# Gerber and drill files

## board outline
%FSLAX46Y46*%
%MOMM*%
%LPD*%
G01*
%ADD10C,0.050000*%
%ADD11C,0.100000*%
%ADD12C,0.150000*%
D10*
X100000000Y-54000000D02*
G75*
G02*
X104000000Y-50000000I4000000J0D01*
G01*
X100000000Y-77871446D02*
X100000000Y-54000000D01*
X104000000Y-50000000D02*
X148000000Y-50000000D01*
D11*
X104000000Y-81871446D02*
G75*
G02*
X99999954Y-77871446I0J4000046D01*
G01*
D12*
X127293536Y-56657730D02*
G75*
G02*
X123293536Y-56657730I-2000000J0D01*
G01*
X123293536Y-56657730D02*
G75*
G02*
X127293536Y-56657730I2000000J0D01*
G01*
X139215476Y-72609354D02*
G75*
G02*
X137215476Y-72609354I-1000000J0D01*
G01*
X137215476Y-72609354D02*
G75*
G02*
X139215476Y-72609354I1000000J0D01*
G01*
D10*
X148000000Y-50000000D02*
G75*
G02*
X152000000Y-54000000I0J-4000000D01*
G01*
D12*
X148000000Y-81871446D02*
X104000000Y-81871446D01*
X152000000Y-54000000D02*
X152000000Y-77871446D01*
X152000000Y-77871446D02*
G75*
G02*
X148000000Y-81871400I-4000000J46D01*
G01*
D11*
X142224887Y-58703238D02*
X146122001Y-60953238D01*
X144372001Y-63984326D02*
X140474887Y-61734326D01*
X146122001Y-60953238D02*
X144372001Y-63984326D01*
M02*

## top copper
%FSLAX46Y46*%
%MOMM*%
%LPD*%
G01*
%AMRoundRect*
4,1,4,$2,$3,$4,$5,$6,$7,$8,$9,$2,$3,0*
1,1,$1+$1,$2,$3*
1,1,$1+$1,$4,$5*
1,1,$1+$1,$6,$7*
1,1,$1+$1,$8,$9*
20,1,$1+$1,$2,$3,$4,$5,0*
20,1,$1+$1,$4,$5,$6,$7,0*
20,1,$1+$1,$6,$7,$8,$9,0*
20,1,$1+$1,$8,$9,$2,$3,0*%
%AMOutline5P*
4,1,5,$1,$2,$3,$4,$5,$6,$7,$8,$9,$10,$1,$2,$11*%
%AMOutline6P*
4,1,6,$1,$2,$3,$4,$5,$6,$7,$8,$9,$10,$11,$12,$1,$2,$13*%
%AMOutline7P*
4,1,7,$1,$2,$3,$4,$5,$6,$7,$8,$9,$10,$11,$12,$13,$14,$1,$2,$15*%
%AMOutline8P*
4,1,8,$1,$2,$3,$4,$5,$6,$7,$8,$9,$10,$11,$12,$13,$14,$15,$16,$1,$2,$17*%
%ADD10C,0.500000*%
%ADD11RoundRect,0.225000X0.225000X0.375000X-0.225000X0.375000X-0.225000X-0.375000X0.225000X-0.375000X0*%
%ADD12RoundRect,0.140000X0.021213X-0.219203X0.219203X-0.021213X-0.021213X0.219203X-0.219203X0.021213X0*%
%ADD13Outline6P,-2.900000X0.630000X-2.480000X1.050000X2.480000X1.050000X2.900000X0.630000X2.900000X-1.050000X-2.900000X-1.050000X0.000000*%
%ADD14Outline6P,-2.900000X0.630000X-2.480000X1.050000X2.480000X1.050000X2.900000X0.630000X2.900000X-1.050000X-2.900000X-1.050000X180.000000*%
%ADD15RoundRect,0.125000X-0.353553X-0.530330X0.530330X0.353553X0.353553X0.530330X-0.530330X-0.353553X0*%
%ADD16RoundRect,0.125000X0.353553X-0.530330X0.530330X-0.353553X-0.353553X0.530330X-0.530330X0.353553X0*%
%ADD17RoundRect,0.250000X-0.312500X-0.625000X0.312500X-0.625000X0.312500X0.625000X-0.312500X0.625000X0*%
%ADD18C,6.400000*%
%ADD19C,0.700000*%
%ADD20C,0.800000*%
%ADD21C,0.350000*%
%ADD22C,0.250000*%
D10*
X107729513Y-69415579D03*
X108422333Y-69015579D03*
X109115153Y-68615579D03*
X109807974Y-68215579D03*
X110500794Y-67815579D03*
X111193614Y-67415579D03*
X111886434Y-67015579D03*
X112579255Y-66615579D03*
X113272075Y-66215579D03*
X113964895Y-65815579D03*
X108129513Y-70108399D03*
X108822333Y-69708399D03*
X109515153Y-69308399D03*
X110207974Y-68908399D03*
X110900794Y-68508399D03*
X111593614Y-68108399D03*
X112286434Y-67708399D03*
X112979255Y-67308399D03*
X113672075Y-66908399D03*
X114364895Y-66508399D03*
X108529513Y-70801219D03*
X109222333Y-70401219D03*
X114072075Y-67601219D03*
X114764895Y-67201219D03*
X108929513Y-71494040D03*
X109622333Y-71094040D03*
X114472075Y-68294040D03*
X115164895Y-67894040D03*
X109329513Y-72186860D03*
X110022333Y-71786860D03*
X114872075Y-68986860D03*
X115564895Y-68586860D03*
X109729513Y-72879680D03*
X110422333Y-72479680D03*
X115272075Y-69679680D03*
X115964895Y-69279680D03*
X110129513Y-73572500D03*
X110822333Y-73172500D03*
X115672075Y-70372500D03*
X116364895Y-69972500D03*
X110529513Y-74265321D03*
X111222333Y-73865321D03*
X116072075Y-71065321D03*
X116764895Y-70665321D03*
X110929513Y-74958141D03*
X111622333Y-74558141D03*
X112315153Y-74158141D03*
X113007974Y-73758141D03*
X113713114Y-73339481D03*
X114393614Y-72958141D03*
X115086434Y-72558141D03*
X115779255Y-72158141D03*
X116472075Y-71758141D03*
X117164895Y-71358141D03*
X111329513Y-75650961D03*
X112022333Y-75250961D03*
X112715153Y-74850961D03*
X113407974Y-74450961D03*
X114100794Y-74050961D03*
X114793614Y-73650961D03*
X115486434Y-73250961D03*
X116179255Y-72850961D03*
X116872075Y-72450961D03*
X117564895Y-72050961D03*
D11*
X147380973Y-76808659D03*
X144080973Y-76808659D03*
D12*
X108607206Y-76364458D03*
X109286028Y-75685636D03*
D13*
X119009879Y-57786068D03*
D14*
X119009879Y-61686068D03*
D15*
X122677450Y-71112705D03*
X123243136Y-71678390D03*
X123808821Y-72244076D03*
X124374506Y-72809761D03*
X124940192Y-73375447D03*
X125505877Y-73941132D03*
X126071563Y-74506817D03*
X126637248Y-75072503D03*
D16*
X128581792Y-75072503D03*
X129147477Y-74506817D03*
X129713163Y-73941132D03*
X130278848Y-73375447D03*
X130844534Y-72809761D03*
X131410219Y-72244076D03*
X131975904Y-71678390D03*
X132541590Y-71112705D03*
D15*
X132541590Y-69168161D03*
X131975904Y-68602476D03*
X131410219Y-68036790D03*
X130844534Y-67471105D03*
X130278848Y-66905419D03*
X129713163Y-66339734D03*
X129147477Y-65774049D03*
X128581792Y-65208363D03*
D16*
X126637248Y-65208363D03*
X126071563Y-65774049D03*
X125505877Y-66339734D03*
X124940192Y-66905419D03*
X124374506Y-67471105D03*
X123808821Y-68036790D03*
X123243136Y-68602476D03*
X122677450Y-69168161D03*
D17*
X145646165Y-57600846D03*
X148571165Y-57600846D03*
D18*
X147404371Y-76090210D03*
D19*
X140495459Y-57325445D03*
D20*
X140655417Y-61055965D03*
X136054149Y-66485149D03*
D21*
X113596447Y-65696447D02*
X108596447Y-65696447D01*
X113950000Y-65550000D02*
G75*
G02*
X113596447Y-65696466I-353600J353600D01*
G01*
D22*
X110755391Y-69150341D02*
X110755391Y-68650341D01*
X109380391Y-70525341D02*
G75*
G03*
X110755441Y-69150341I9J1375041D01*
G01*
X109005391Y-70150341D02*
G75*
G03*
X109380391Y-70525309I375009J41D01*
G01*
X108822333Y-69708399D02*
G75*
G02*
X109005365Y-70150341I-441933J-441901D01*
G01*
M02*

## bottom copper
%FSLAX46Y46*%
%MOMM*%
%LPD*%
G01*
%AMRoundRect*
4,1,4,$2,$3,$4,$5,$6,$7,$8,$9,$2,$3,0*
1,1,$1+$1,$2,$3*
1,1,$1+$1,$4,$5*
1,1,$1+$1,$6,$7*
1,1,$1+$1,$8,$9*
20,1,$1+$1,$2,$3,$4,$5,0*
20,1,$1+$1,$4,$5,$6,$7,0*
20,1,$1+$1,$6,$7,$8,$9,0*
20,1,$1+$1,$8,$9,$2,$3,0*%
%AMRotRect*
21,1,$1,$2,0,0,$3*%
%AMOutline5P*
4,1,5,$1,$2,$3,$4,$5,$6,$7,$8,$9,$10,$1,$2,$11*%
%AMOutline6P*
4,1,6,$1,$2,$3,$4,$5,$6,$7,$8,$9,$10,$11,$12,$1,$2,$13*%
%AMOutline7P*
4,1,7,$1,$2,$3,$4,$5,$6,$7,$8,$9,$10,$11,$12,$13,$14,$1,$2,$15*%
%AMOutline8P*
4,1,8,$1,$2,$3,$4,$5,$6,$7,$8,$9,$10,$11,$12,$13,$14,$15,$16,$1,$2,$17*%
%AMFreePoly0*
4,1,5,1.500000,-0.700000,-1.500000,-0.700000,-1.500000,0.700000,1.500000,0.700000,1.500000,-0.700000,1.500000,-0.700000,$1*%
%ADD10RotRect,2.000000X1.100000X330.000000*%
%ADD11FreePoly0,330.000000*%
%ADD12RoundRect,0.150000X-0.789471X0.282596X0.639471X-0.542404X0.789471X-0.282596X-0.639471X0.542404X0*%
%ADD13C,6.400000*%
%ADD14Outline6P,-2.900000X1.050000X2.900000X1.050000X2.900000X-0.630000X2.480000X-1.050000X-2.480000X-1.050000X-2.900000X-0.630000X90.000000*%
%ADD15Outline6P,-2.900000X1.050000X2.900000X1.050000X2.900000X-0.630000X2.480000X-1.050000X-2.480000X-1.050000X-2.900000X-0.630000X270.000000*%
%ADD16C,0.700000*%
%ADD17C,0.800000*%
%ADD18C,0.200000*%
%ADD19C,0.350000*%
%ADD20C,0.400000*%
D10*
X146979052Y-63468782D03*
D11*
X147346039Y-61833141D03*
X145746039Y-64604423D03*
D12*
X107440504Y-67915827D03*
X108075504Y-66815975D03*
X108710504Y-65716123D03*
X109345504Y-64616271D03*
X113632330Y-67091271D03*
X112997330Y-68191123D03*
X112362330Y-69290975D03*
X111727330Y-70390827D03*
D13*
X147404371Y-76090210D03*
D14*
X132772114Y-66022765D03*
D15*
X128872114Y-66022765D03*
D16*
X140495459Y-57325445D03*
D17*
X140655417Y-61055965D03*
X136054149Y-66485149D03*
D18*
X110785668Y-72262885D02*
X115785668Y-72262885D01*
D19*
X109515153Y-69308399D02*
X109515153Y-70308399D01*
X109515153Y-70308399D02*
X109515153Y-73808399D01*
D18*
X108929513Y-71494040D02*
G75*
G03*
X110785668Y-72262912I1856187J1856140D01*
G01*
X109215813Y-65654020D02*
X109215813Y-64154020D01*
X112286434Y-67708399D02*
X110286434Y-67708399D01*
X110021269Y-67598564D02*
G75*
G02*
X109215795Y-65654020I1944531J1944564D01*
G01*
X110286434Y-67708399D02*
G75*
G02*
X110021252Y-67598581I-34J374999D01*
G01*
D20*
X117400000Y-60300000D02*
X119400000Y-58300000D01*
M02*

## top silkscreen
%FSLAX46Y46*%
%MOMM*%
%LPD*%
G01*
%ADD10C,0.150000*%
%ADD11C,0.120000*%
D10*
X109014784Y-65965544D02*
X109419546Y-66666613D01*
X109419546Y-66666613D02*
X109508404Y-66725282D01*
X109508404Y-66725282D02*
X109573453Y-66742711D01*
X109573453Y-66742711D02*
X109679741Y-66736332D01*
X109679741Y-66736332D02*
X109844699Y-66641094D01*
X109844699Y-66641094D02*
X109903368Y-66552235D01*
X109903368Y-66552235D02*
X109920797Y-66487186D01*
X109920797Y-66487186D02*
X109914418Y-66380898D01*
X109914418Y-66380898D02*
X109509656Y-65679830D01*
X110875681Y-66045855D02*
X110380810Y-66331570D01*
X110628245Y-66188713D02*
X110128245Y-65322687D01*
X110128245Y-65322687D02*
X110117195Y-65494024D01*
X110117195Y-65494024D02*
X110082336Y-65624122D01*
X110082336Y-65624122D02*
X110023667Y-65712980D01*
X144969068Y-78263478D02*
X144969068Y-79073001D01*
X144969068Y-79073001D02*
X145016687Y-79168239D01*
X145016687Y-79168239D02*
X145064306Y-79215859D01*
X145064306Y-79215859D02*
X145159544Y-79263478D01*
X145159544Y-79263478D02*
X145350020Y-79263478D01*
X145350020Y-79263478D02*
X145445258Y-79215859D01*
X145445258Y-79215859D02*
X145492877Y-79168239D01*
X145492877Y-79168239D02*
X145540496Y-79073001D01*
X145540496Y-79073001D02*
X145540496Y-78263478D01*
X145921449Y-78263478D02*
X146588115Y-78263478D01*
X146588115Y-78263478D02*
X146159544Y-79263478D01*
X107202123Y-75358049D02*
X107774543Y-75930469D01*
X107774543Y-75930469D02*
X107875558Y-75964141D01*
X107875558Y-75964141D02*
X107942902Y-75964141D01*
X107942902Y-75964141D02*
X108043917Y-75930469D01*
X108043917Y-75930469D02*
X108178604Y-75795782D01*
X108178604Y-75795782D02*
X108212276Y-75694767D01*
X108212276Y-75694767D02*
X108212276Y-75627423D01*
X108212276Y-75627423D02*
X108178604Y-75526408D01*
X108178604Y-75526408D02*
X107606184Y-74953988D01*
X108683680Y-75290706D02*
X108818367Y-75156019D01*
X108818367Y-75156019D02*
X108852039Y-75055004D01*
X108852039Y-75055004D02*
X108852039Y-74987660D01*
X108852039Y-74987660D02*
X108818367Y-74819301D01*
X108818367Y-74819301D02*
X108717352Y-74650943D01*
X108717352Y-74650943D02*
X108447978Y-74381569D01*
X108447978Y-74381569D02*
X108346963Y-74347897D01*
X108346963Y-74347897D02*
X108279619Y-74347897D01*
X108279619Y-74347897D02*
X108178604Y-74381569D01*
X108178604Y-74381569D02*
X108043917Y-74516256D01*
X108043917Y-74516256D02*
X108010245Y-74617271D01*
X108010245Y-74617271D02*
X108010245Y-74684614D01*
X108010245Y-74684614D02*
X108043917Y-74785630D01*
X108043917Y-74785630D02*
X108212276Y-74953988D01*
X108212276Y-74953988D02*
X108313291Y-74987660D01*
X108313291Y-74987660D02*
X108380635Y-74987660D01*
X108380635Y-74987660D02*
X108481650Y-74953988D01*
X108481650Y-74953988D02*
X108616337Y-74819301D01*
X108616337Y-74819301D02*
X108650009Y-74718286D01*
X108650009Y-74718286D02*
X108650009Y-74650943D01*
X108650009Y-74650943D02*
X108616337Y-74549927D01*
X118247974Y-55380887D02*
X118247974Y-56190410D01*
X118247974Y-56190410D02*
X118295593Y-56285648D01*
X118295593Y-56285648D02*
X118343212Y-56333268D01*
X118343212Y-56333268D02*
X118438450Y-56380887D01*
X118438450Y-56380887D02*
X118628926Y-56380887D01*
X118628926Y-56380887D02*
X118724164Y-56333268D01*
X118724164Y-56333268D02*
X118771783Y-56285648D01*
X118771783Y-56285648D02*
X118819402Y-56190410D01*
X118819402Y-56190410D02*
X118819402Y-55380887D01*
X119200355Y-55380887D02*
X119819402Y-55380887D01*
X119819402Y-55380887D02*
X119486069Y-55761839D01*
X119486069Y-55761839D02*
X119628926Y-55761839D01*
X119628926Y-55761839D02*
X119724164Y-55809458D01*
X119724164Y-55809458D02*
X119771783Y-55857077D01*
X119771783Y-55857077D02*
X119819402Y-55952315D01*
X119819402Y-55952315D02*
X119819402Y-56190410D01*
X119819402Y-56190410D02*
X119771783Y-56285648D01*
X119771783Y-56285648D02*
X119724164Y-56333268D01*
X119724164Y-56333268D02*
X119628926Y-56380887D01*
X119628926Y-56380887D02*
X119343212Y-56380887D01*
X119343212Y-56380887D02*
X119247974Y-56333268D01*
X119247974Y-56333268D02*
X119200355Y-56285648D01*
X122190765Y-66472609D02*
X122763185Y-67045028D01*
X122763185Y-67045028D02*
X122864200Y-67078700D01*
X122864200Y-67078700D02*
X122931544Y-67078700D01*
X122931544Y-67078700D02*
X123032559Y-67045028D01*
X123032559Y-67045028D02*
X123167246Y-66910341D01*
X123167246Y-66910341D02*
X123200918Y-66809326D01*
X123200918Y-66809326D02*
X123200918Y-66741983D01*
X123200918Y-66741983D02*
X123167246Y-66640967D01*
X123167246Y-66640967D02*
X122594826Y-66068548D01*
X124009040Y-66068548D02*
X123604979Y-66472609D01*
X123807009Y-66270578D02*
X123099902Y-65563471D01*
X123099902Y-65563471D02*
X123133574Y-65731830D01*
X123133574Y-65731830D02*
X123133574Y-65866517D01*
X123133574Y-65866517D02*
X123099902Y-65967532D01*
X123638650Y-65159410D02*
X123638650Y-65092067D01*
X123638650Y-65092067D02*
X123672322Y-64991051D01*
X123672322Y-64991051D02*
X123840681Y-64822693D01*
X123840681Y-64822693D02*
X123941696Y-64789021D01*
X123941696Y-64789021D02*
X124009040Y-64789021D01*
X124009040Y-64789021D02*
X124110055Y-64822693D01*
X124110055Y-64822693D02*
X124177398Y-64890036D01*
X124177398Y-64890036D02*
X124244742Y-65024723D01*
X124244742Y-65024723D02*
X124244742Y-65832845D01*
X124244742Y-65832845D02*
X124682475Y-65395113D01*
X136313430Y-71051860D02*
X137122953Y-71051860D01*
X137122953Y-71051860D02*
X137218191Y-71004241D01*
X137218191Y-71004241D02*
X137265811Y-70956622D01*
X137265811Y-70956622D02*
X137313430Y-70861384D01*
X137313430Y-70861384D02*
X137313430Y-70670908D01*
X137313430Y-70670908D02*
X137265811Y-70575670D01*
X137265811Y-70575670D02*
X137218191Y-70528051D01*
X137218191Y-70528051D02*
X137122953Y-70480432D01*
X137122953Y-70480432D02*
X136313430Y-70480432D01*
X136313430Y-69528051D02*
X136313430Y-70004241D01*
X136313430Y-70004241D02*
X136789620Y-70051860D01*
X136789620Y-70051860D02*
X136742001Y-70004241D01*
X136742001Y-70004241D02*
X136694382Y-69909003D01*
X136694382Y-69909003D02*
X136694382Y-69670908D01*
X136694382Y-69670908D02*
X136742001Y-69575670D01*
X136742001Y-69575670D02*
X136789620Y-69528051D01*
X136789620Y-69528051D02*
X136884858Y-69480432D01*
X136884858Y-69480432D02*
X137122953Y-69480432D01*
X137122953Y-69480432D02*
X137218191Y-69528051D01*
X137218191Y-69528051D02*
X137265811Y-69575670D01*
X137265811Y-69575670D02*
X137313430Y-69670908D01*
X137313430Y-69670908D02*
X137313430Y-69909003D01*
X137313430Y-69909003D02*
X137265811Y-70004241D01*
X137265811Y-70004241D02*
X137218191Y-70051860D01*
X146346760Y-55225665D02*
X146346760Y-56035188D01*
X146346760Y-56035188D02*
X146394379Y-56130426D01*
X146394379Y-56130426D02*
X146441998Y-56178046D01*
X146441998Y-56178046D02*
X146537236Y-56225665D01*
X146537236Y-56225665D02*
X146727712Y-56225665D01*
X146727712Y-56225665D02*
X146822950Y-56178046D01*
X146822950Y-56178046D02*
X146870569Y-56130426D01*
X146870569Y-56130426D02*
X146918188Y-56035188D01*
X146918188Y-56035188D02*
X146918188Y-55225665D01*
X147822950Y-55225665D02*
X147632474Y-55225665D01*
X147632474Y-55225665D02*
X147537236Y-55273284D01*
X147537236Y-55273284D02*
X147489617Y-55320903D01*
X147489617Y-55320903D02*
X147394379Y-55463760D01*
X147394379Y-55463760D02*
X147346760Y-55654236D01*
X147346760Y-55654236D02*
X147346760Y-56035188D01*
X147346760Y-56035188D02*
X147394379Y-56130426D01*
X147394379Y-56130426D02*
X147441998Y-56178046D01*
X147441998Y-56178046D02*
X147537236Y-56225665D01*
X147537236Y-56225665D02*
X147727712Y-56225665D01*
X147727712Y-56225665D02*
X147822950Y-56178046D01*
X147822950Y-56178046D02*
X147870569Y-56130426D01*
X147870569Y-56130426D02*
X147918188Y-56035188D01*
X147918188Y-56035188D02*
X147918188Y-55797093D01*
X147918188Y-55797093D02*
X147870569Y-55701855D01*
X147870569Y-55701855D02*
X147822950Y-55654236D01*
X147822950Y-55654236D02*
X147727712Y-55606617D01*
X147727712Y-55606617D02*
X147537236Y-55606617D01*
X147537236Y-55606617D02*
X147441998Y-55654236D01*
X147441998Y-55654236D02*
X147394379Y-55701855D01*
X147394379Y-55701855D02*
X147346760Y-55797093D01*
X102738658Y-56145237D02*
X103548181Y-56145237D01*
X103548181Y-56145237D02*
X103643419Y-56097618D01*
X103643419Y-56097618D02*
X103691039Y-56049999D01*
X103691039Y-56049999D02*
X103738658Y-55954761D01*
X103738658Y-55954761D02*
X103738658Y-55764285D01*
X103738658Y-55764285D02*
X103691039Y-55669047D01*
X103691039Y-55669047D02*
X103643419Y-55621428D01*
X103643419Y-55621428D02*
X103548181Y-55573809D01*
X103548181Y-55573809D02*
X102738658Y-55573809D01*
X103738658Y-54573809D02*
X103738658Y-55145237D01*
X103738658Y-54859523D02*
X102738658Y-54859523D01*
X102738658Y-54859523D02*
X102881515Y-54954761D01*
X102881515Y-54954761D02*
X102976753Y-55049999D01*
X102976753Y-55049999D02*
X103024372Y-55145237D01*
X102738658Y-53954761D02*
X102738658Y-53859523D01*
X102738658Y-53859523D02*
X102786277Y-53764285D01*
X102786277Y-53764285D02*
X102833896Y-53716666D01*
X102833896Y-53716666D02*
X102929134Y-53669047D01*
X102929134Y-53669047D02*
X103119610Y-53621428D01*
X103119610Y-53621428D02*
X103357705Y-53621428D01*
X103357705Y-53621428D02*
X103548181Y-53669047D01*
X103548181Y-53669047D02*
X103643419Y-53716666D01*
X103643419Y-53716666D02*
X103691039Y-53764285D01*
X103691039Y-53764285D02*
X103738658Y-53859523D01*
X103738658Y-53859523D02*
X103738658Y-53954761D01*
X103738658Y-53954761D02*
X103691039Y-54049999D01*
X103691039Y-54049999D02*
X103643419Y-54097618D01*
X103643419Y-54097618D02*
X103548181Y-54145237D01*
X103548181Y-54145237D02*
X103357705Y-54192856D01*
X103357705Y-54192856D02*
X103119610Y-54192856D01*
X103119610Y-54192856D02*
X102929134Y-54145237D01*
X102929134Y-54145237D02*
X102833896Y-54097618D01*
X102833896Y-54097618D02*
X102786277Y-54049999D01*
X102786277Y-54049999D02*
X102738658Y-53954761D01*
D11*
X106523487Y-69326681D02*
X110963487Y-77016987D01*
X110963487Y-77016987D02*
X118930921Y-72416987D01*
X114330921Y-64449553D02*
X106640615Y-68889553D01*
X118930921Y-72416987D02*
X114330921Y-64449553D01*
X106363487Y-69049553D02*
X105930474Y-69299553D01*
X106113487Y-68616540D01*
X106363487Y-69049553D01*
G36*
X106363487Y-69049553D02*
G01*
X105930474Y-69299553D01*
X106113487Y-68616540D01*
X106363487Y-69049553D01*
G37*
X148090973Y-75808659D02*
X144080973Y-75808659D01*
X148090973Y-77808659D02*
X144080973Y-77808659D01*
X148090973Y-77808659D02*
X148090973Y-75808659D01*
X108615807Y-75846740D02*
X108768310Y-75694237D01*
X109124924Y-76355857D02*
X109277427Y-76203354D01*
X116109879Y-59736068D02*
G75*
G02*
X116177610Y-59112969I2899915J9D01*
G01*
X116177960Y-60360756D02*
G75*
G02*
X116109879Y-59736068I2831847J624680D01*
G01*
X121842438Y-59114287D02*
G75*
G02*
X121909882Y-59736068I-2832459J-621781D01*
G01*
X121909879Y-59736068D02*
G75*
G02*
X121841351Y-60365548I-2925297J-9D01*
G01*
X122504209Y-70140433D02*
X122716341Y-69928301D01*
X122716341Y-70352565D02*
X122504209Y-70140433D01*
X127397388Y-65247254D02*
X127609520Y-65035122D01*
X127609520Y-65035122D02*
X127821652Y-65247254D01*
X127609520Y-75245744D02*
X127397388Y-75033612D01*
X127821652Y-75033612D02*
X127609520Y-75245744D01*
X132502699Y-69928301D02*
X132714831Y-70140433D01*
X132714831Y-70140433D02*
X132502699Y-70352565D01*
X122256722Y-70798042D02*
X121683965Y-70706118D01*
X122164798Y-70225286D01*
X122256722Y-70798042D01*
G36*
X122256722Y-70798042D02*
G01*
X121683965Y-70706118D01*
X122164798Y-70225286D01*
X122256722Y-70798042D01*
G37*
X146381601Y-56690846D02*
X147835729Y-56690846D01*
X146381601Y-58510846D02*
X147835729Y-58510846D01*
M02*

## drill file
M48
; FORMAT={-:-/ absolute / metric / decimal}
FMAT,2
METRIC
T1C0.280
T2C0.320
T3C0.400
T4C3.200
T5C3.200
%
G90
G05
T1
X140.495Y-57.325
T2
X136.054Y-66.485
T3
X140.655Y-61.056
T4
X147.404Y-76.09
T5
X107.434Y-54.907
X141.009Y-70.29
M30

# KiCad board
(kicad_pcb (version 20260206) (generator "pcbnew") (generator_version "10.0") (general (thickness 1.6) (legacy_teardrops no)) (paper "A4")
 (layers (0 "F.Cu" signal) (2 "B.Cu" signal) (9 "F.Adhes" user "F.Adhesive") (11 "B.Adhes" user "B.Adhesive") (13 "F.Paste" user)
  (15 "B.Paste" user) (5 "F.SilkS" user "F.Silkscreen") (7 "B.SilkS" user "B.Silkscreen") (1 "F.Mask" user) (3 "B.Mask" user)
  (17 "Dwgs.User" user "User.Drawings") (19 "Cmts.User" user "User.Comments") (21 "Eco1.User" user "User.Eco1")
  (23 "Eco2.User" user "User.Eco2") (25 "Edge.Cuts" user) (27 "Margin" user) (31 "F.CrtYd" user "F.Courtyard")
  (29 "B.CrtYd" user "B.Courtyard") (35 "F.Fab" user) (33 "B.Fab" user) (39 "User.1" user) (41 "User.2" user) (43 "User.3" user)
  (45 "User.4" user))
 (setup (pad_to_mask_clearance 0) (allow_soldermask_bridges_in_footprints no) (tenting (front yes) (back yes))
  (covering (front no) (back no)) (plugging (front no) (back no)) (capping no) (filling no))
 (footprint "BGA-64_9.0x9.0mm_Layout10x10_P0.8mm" (layer "F.Cu") (at 112.647204 70.73327 30)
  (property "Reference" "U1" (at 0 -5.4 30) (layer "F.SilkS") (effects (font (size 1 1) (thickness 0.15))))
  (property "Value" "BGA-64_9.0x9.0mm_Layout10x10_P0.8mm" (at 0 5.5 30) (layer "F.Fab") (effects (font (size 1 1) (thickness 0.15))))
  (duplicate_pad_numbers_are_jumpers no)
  (fp_line (start -4.6 -4.28) (end -4.6 4.6) (stroke (width 0.12) (type solid)) (layer "F.SilkS"))
  (fp_line (start -4.6 4.6) (end 4.6 4.6) (stroke (width 0.12) (type solid)) (layer "F.SilkS"))
  (fp_line (start 4.6 -4.6) (end -4.28 -4.6) (stroke (width 0.12) (type solid)) (layer "F.SilkS"))
  (fp_line (start 4.6 4.6) (end 4.6 -4.6) (stroke (width 0.12) (type solid)) (layer "F.SilkS"))
  (fp_poly
   (pts (xy -4.6 -4.6) (xy -5.1 -4.6) (xy -4.6 -5.1) (xy -4.6 -4.6)) (stroke (width 0.12) (type solid)) (fill yes) (layer "F.SilkS"))
  (pad "A1" smd circle (at -3.6 -3.599999 30) (size 0.5 0.5) (layers "F.Cu" "F.Mask" "F.Paste") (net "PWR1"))
  (pad "A2" smd circle (at -2.8 -3.6 30) (size 0.5 0.5) (layers "F.Cu" "F.Mask" "F.Paste") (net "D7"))
  (pad "A3" smd circle (at -2 -3.6 30) (size 0.5 0.5) (layers "F.Cu" "F.Mask" "F.Paste") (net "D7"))
  (pad "A4" smd circle (at -1.2 -3.599999 30) (size 0.5 0.5) (layers "F.Cu" "F.Mask" "F.Paste") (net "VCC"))
  (pad "A5" smd circle (at -0.4 -3.6 30) (size 0.5 0.5) (layers "F.Cu" "F.Mask" "F.Paste"))
  (pad "A6" smd circle (at 0.4 -3.6 30) (size 0.5 0.5) (layers "F.Cu" "F.Mask" "F.Paste") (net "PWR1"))
  (pad "A7" smd circle (at 1.199999 -3.6 30) (size 0.5 0.5) (layers "F.Cu" "F.Mask" "F.Paste") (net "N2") (clearance 0.1))
  (pad "A8" smd circle (at 2 -3.6 30) (size 0.5 0.5) (layers "F.Cu" "F.Mask" "F.Paste"))
  (pad "A9" smd circle (at 2.8 -3.6 30) (size 0.5 0.5) (layers "F.Cu" "F.Mask" "F.Paste") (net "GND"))
  (pad "A10" smd circle (at 3.599999 -3.6 30) (size 0.5 0.5) (layers "F.Cu" "F.Mask" "F.Paste") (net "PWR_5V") (clearance 0.1))
  (pad "B1" smd circle (at -3.6 -2.8 30) (size 0.5 0.5) (layers "F.Cu" "F.Mask" "F.Paste") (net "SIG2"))
  (pad "B2" smd circle (at -2.8 -2.8 30) (size 0.5 0.5) (layers "F.Cu" "F.Mask" "F.Paste") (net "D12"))
  (pad "B3" smd circle (at -2 -2.8 30) (size 0.5 0.5) (layers "F.Cu" "F.Mask" "F.Paste") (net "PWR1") (clearance 0.1))
  (pad "B4" smd circle (at -1.2 -2.8 30) (size 0.5 0.5) (layers "F.Cu" "F.Mask" "F.Paste") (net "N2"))
  (pad "B5" smd circle (at -0.4 -2.8 30) (size 0.5 0.5) (layers "F.Cu" "F.Mask" "F.Paste") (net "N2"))
  (pad "B6" smd circle (at 0.4 -2.8 30) (size 0.5 0.5) (layers "F.Cu" "F.Mask" "F.Paste") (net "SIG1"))
  (pad "B7" smd circle (at 1.2 -2.8 30) (size 0.5 0.5) (layers "F.Cu" "F.Mask" "F.Paste") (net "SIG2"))
  (pad "B8" smd circle (at 2 -2.8 30) (size 0.5 0.5) (layers "F.Cu" "F.Mask" "F.Paste") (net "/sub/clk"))
  (pad "B9" smd circle (at 2.8 -2.8 30) (size 0.5 0.5) (layers "F.Cu" "F.Mask" "F.Paste") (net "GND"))
  (pad "B10" smd circle (at 3.6 -2.8 30) (size 0.5 0.5) (layers "F.Cu" "F.Mask" "F.Paste") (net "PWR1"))
  (pad "C1" smd circle (at -3.6 -2 30) (size 0.5 0.5) (layers "F.Cu" "F.Mask" "F.Paste"))
  (pad "C2" smd circle (at -2.8 -2 30) (size 0.5 0.5) (layers "F.Cu" "F.Mask" "F.Paste"))
  (pad "C9" smd circle (at 2.8 -2 30) (size 0.5 0.5) (layers "F.Cu" "F.Mask" "F.Paste") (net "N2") (clearance 0.1))
  (pad "C10" smd circle (at 3.6 -2 30) (size 0.5 0.5) (layers "F.Cu" "F.Mask" "F.Paste") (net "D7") (clearance 0.35))
  (pad "D1" smd circle (at -3.6 -1.199999 30) (size 0.5 0.5) (layers "F.Cu" "F.Mask" "F.Paste") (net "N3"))
  (pad "D2" smd circle (at -2.8 -1.2 30) (size 0.5 0.5) (layers "F.Cu" "F.Mask" "F.Paste") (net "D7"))
  (pad "D9" smd circle (at 2.8 -1.2 30) (size 0.5 0.5) (layers "F.Cu" "F.Mask" "F.Paste") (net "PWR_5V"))
  (pad "D10" smd circle (at 3.599999 -1.2 30) (size 0.5 0.5) (layers "F.Cu" "F.Mask" "F.Paste") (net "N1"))
  (pad "E1" smd circle (at -3.6 -0.4 30) (size 0.5 0.5) (layers "F.Cu" "F.Mask" "F.Paste") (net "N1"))
  (pad "E2" smd circle (at -2.8 -0.4 30) (size 0.5 0.5) (layers "F.Cu" "F.Mask" "F.Paste") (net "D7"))
  (pad "E9" smd circle (at 2.8 -0.4 30) (size 0.5 0.5) (layers "F.Cu" "F.Mask" "F.Paste") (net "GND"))
  (pad "E10" smd circle (at 3.6 -0.4 30) (size 0.5 0.5) (layers "F.Cu" "F.Mask" "F.Paste") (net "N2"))
  (pad "F1" smd circle (at -3.6 0.4 30) (size 0.5 0.5) (layers "F.Cu" "F.Mask" "F.Paste") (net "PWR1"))
  (pad "F2" smd circle (at -2.8 0.4 30) (size 0.5 0.5) (layers "F.Cu" "F.Mask" "F.Paste") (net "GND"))
  (pad "F9" smd circle (at 2.8 0.4 30) (size 0.5 0.5) (layers "F.Cu" "F.Mask" "F.Paste") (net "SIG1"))
  (pad "F10" smd circle (at 3.6 0.4 30) (size 0.5 0.5) (layers "F.Cu" "F.Mask" "F.Paste") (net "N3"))
  (pad "G1" smd circle (at -3.599999 1.2 30) (size 0.5 0.5) (layers "F.Cu" "F.Mask" "F.Paste") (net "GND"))
  (pad "G2" smd circle (at -2.8 1.2 30) (size 0.5 0.5) (layers "F.Cu" "F.Mask" "F.Paste") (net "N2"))
  (pad "G9" smd circle (at 2.8 1.2 30) (size 0.5 0.5) (layers "F.Cu" "F.Mask" "F.Paste") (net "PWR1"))
  (pad "G10" smd circle (at 3.6 1.199999 30) (size 0.5 0.5) (layers "F.Cu" "F.Mask" "F.Paste"))
  (pad "H1" smd circle (at -3.6 2 30) (size 0.5 0.5) (layers "F.Cu" "F.Mask" "F.Paste") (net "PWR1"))
  (pad "H2" smd circle (at -2.8 2 30) (size 0.5 0.5) (layers "F.Cu" "F.Mask" "F.Paste") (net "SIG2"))
  (pad "H9" smd circle (at 2.8 2 30) (size 0.5 0.5) (layers "F.Cu" "F.Mask" "F.Paste") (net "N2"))
  (pad "H10" smd circle (at 3.6 2 30) (size 0.5 0.5) (layers "F.Cu" "F.Mask" "F.Paste") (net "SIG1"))
  (pad "J1" smd circle (at -3.6 2.8 30) (size 0.5 0.5) (layers "F.Cu" "F.Mask" "F.Paste") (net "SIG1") (clearance 0.1))
  (pad "J2" smd circle (at -2.8 2.8 30) (size 0.5 0.5) (layers "F.Cu" "F.Mask" "F.Paste") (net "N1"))
  (pad "J3" smd circle (at -2 2.8 30) (size 0.5 0.5) (layers "F.Cu" "F.Mask" "F.Paste"))
  (pad "J4" smd circle (at -1.2 2.8 30) (size 0.5 0.5) (layers "F.Cu" "F.Mask" "F.Paste") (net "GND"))
  (pad "J5" smd circle (at -0.38 2.79 30) (size 0.5 0.5) (layers "F.Cu" "F.Mask" "F.Paste") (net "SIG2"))
  (pad "J6" smd circle (at 0.4 2.8 30) (size 0.5 0.5) (layers "F.Cu" "F.Mask" "F.Paste"))
  (pad "J7" smd circle (at 1.2 2.8 30) (size 0.5 0.5) (layers "F.Cu" "F.Mask" "F.Paste") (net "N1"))
  (pad "J8" smd circle (at 2 2.8 30) (size 0.5 0.5) (layers "F.Cu" "F.Mask" "F.Paste"))
  (pad "J9" smd circle (at 2.8 2.8 30) (size 0.5 0.5) (layers "F.Cu" "F.Mask" "F.Paste") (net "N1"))
  (pad "J10" smd circle (at 3.6 2.8 30) (size 0.5 0.5) (layers "F.Cu" "F.Mask" "F.Paste") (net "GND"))
  (pad "K1" smd circle (at -3.599999 3.6 30) (size 0.5 0.5) (layers "F.Cu" "F.Mask" "F.Paste") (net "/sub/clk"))
  (pad "K2" smd circle (at -2.8 3.6 30) (size 0.5 0.5) (layers "F.Cu" "F.Mask" "F.Paste") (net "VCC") (clearance 0.35))
  (pad "K3" smd circle (at -2 3.6 30) (size 0.5 0.5) (layers "F.Cu" "F.Mask" "F.Paste"))
  (pad "K4" smd circle (at -1.199999 3.6 30) (size 0.5 0.5) (layers "F.Cu" "F.Mask" "F.Paste") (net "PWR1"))
  (pad "K5" smd circle (at -0.4 3.6 30) (size 0.5 0.5) (layers "F.Cu" "F.Mask" "F.Paste") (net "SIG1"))
  (pad "K6" smd circle (at 0.4 3.6 30) (size 0.5 0.5) (layers "F.Cu" "F.Mask" "F.Paste") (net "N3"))
  (pad "K7" smd circle (at 1.2 3.599999 30) (size 0.5 0.5) (layers "F.Cu" "F.Mask" "F.Paste") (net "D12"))
  (pad "K8" smd circle (at 2 3.6 30) (size 0.5 0.5) (layers "F.Cu" "F.Mask" "F.Paste") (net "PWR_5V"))
  (pad "K9" smd circle (at 2.8 3.6 30) (size 0.5 0.5) (layers "F.Cu" "F.Mask" "F.Paste") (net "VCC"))
  (pad "K10" smd circle (at 3.6 3.599999 30) (size 0.5 0.5) (layers "F.Cu" "F.Mask" "F.Paste")))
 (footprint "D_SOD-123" (layer "F.Cu") (at 145.730973 76.808659 180)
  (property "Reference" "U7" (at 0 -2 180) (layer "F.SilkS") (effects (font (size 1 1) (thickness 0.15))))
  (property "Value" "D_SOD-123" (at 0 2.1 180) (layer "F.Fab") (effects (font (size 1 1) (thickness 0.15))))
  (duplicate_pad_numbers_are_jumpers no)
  (fp_line (start -2.36 1) (end 1.65 1) (stroke (width 0.12) (type solid)) (layer "F.SilkS"))
  (fp_line (start -2.36 -1) (end 1.65 -1) (stroke (width 0.12) (type solid)) (layer "F.SilkS"))
  (fp_line (start -2.36 -1) (end -2.36 1) (stroke (width 0.12) (type solid)) (layer "F.SilkS"))
  (pad "1" smd roundrect (at -1.65 0 180) (size 0.9 1.2) (layers "F.Cu" "F.Mask" "F.Paste") (roundrect_rratio 0.25) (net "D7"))
  (pad "2" smd roundrect (at 1.65 0 180) (size 0.9 1.2) (layers "F.Cu" "F.Mask" "F.Paste") (roundrect_rratio 0.25) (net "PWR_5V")
   (clearance 0.35)))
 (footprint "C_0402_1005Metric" (layer "F.Cu") (at 108.946617 76.025047 45)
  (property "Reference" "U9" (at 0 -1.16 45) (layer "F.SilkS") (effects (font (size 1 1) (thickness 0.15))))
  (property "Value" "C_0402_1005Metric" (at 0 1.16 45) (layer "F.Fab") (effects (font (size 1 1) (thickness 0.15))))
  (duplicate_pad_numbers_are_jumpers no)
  (fp_line (start -0.107836 -0.36) (end 0.107836 -0.36) (stroke (width 0.12) (type solid)) (layer "F.SilkS"))
  (fp_line (start -0.107836 0.36) (end 0.107836 0.36) (stroke (width 0.12) (type solid)) (layer "F.SilkS"))
  (pad "1" smd roundrect (at -0.48 0 45) (size 0.56 0.62) (layers "F.Cu" "F.Mask" "F.Paste") (roundrect_rratio 0.25))
  (pad "2" smd roundrect (at 0.48 0 45) (size 0.56 0.62) (layers "F.Cu" "F.Mask" "F.Paste") (roundrect_rratio 0.25) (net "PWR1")
   (clearance 0.1)))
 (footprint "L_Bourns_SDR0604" (layer "F.Cu") (at 119.009879 59.736068)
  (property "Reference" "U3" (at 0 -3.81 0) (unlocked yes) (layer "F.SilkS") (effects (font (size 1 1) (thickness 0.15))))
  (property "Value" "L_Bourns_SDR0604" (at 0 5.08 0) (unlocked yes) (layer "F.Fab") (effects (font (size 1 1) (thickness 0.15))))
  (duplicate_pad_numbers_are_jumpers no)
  (fp_arc (start -2.9 0) (mid -2.883018 -0.313385) (end -2.832269 -0.623099) (stroke (width 0.12) (type default)) (layer "F.SilkS"))
  (fp_arc (start -2.831919 0.624688) (mid -2.88293 0.314193) (end -2.9 0) (stroke (width 0.12) (type default)) (layer "F.SilkS"))
  (fp_arc (start 2.832559 -0.621781) (mid 2.883091 -0.312714) (end 2.9 0) (stroke (width 0.12) (type default)) (layer "F.SilkS"))
  (fp_arc (start 2.9 0) (mid 2.882818 0.3166) (end 2.831472 0.62948) (stroke (width 0.12) (type default)) (layer "F.SilkS"))
  (pad "1" smd roundrect (at 0 -1.95) (size 5.8 2.1) (layers "F.Cu" "F.Mask" "F.Paste") (roundrect_rratio 0) (chamfer_ratio 0.2)
   (chamfer top_left top_right) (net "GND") (die_length 2))
  (pad "2" smd roundrect (at 0 1.95 180) (size 5.8 2.1) (layers "F.Cu" "F.Mask" "F.Paste") (roundrect_rratio 0) (chamfer_ratio 0.2)
   (chamfer top_left top_right) (die_length 2)))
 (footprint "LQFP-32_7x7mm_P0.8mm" (layer "F.Cu") (at 127.60952 70.140433 45)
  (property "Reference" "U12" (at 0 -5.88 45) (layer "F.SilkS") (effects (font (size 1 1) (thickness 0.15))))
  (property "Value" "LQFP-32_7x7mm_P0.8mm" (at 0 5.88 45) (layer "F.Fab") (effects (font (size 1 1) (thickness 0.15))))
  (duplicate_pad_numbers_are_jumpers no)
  (fp_line (start -3.61 -3.61) (end -3.31 -3.61) (stroke (width 0.12) (type solid)) (layer "F.SilkS"))
  (fp_line (start -3.61 -3.31) (end -3.61 -3.61) (stroke (width 0.12) (type solid)) (layer "F.SilkS"))
  (fp_line (start 3.31 -3.61) (end 3.61 -3.61) (stroke (width 0.12) (type solid)) (layer "F.SilkS"))
  (fp_line (start 3.61 -3.61) (end 3.61 -3.31) (stroke (width 0.12) (type solid)) (layer "F.SilkS"))
  (fp_line (start -3.61 3.61) (end -3.61 3.31) (stroke (width 0.12) (type solid)) (layer "F.SilkS"))
  (fp_line (start -3.31 3.61) (end -3.61 3.61) (stroke (width 0.12) (type solid)) (layer "F.SilkS"))
  (fp_line (start 3.61 3.31) (end 3.61 3.61) (stroke (width 0.12) (type solid)) (layer "F.SilkS"))
  (fp_line (start 3.61 3.61) (end 3.31 3.61) (stroke (width 0.12) (type solid)) (layer "F.SilkS"))
  (fp_poly (pts (xy -4.25 -3.32) (xy -4.59 -3.79) (xy -3.91 -3.79)) (stroke (width 0.12) (type solid)) (fill yes) (layer "F.SilkS"))
  (pad "1" smd roundrect (at -4.175 -2.8 45) (size 1.5 0.5) (layers "F.Cu" "F.Mask" "F.Paste") (roundrect_rratio 0.25))
  (pad "2" smd roundrect (at -4.175 -2 45) (size 1.5 0.5) (layers "F.Cu" "F.Mask" "F.Paste") (roundrect_rratio 0.25))
  (pad "3" smd roundrect (at -4.175 -1.2 45) (size 1.5 0.5) (layers "F.Cu" "F.Mask" "F.Paste") (roundrect_rratio 0.25) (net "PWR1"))
  (pad "4" smd roundrect (at -4.175 -0.4 45) (size 1.5 0.5) (layers "F.Cu" "F.Mask" "F.Paste") (roundrect_rratio 0.25) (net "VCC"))
  (pad "5" smd roundrect (at -4.175 0.4 45) (size 1.5 0.5) (layers "F.Cu" "F.Mask" "F.Paste") (roundrect_rratio 0.25) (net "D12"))
  (pad "6" smd roundrect (at -4.175 1.2 45) (size 1.5 0.5) (layers "F.Cu" "F.Mask" "F.Paste") (roundrect_rratio 0.25) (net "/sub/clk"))
  (pad "7" smd roundrect (at -4.175 2 45) (size 1.5 0.5) (layers "F.Cu" "F.Mask" "F.Paste") (roundrect_rratio 0.25) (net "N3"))
  (pad "8" smd roundrect (at -4.175 2.8 45) (size 1.5 0.5) (layers "F.Cu" "F.Mask" "F.Paste") (roundrect_rratio 0.25) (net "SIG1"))
  (pad "9" smd roundrect (at -2.8 4.175 45) (size 0.5 1.5) (layers "F.Cu" "F.Mask" "F.Paste") (roundrect_rratio 0.25))
  (pad "10" smd roundrect (at -2 4.175 45) (size 0.5 1.5) (layers "F.Cu" "F.Mask" "F.Paste") (roundrect_rratio 0.25))
  (pad "11" smd roundrect (at -1.2 4.175 45) (size 0.5 1.5) (layers "F.Cu" "F.Mask" "F.Paste") (roundrect_rratio 0.25))
  (pad "12" smd roundrect (at -0.4 4.175 45) (size 0.5 1.5) (layers "F.Cu" "F.Mask" "F.Paste") (roundrect_rratio 0.25) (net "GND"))
  (pad "13" smd roundrect (at 0.4 4.175 45) (size 0.5 1.5) (layers "F.Cu" "F.Mask" "F.Paste") (roundrect_rratio 0.25) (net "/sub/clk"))
  (pad "14" smd roundrect (at 1.2 4.175 45) (size 0.5 1.5) (layers "F.Cu" "F.Mask" "F.Paste") (roundrect_rratio 0.25) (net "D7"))
  (pad "15" smd roundrect (at 2 4.175 45) (size 0.5 1.5) (layers "F.Cu" "F.Mask" "F.Paste") (roundrect_rratio 0.25) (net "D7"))
  (pad "16" smd roundrect (at 2.8 4.175 45) (size 0.5 1.5) (layers "F.Cu" "F.Mask" "F.Paste") (roundrect_rratio 0.25) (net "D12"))
  (pad "17" smd roundrect (at 4.175 2.8 45) (size 1.5 0.5) (layers "F.Cu" "F.Mask" "F.Paste") (roundrect_rratio 0.25) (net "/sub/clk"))
  (pad "18" smd roundrect (at 4.175 2 45) (size 1.5 0.5) (layers "F.Cu" "F.Mask" "F.Paste") (roundrect_rratio 0.25) (clearance 0.35))
  (pad "19" smd roundrect (at 4.175 1.2 45) (size 1.5 0.5) (layers "F.Cu" "F.Mask" "F.Paste") (roundrect_rratio 0.25))
  (pad "20" smd roundrect (at 4.175 0.4 45) (size 1.5 0.5) (layers "F.Cu" "F.Mask" "F.Paste") (roundrect_rratio 0.25) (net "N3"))
  (pad "21" smd roundrect (at 4.175 -0.4 45) (size 1.5 0.5) (layers "F.Cu" "F.Mask" "F.Paste") (roundrect_rratio 0.25) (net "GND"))
  (pad "22" smd roundrect (at 4.175 -1.2 45) (size 1.5 0.5) (layers "F.Cu" "F.Mask" "F.Paste") (roundrect_rratio 0.25) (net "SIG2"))
  (pad "23" smd roundrect (at 4.175 -2 45) (size 1.5 0.5) (layers "F.Cu" "F.Mask" "F.Paste") (roundrect_rratio 0.25))
  (pad "24" smd roundrect (at 4.175 -2.8 45) (size 1.5 0.5) (layers "F.Cu" "F.Mask" "F.Paste") (roundrect_rratio 0.25) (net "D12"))
  (pad "25" smd roundrect (at 2.8 -4.175 45) (size 0.5 1.5) (layers "F.Cu" "F.Mask" "F.Paste") (roundrect_rratio 0.25) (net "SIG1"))
  (pad "26" smd roundrect (at 2 -4.175 45) (size 0.5 1.5) (layers "F.Cu" "F.Mask" "F.Paste") (roundrect_rratio 0.25) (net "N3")
   (clearance 0.35))
  (pad "27" smd roundrect (at 1.2 -4.175 45) (size 0.5 1.5) (layers "F.Cu" "F.Mask" "F.Paste") (roundrect_rratio 0.25) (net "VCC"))
  (pad "28" smd roundrect (at 0.4 -4.175 45) (size 0.5 1.5) (layers "F.Cu" "F.Mask" "F.Paste") (roundrect_rratio 0.25) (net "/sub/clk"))
  (pad "29" smd roundrect (at -0.4 -4.175 45) (size 0.5 1.5) (layers "F.Cu" "F.Mask" "F.Paste") (roundrect_rratio 0.25) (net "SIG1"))
  (pad "30" smd roundrect (at -1.2 -4.175 45) (size 0.5 1.5) (layers "F.Cu" "F.Mask" "F.Paste") (roundrect_rratio 0.25))
  (pad "31" smd roundrect (at -2 -4.175 45) (size 0.5 1.5) (layers "F.Cu" "F.Mask" "F.Paste") (roundrect_rratio 0.25) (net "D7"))
  (pad "32" smd roundrect (at -2.8 -4.175 45) (size 0.5 1.5) (layers "F.Cu" "F.Mask" "F.Paste") (roundrect_rratio 0.25) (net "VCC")))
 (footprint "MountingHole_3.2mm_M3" (layer "F.Cu") (at 141.008611 70.289956 90)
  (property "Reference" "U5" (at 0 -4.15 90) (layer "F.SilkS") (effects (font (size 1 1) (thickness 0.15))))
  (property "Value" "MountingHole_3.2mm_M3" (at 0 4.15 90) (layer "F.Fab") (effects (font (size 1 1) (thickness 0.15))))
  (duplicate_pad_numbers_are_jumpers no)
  (pad "" np_thru_hole circle (at 0 0 90) (size 3.2 3.2) (drill 3.2) (layers "*.Cu" "*.Mask")))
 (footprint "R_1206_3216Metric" (layer "F.Cu") (at 147.108665 57.600846)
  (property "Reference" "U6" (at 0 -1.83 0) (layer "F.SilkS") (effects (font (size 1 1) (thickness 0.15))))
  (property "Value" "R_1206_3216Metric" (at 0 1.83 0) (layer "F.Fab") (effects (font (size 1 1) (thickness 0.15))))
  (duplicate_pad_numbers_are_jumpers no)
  (fp_line (start -0.727064 -0.91) (end 0.727064 -0.91) (stroke (width 0.12) (type solid)) (layer "F.SilkS"))
  (fp_line (start -0.727064 0.91) (end 0.727064 0.91) (stroke (width 0.12) (type solid)) (layer "F.SilkS"))
  (pad "1" smd roundrect (at -1.4625 0) (size 1.125 1.75) (layers "F.Cu" "F.Mask" "F.Paste") (roundrect_rratio 0.222222))
  (pad "2" smd roundrect (at 1.4625 0) (size 1.125 1.75) (layers "F.Cu" "F.Mask" "F.Paste") (roundrect_rratio 0.222222) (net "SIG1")))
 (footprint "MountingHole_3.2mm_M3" (layer "F.Cu") (at 107.433839 54.907143 90)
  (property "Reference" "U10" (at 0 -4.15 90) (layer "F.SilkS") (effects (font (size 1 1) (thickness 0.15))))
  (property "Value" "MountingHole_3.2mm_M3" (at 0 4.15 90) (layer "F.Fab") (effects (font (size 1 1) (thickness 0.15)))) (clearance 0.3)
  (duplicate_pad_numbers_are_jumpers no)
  (pad "" np_thru_hole circle (at 0 0 90) (size 3.2 3.2) (drill 3.2) (layers "*.Cu" "*.Mask")))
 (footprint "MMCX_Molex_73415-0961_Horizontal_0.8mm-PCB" (layer "B.Cu") (at 144.597482 62.093782 -30)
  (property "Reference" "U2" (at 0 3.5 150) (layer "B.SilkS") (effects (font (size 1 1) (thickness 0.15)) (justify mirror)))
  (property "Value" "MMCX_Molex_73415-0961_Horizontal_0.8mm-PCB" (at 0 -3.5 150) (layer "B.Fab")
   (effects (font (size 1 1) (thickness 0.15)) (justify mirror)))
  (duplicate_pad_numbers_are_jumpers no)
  (fp_line (start -3.75 -1.75) (end 0.75 -1.75) (stroke (width 0.1) (type solid)) (layer "Edge.Cuts"))
  (fp_line (start 0.75 1.75) (end -3.75 1.749999) (stroke (width 0.1) (type solid)) (layer "Edge.Cuts"))
  (fp_line (start 0.75 -1.75) (end 0.75 1.75) (stroke (width 0.1) (type solid)) (layer "Edge.Cuts"))
  (pad "1" smd rect (at 2.75 0 330) (size 2 1.1) (layers "B.Cu" "B.Mask" "B.Paste") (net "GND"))
  (pad "2" smd custom (at 2.25 -1.6 330) (size 3 1.4) (layers "B.Cu" "B.Mask" "B.Paste") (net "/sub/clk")
   (options (clearance outline) (anchor rect)) (primitives))
  (pad "2" smd custom (at 2.25 1.6 330) (size 3 1.4) (layers "B.Cu" "B.Mask" "B.Paste") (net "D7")
   (options (clearance outline) (anchor rect)) (primitives)))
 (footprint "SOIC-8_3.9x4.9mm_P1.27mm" (layer "B.Cu") (at 110.536417 67.503549 -30)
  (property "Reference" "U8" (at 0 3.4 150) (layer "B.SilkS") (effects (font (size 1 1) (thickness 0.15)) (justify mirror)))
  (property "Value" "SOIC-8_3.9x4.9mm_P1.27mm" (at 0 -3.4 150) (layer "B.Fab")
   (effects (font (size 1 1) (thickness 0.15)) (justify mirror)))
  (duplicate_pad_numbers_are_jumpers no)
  (pad "1" smd roundrect (at -2.475 1.905 330) (size 1.95 0.6) (layers "B.Cu" "B.Mask" "B.Paste") (roundrect_rratio 0.25))
  (pad "2" smd roundrect (at -2.475 0.635 330) (size 1.95 0.6) (layers "B.Cu" "B.Mask" "B.Paste") (roundrect_rratio 0.25))
  (pad "3" smd roundrect (at -2.475 -0.635 330) (size 1.95 0.6) (layers "B.Cu" "B.Mask" "B.Paste") (roundrect_rratio 0.25) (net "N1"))
  (pad "4" smd roundrect (at -2.475 -1.905 330) (size 1.95 0.6) (layers "B.Cu" "B.Mask" "B.Paste") (roundrect_rratio 0.25) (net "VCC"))
  (pad "5" smd roundrect (at 2.475 -1.905 330) (size 1.95 0.6) (layers "B.Cu" "B.Mask" "B.Paste") (roundrect_rratio 0.25))
  (pad "6" smd roundrect (at 2.475 -0.635 330) (size 1.95 0.6) (layers "B.Cu" "B.Mask" "B.Paste") (roundrect_rratio 0.25) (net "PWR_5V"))
  (pad "7" smd roundrect (at 2.475 0.635 330) (size 1.95 0.6) (layers "B.Cu" "B.Mask" "B.Paste") (roundrect_rratio 0.25) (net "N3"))
  (pad "8" smd roundrect (at 2.475 1.905 330) (size 1.95 0.6) (layers "B.Cu" "B.Mask" "B.Paste") (roundrect_rratio 0.25) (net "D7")))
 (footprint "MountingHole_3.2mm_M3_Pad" (layer "B.Cu") (at 147.404371 76.09021 -30)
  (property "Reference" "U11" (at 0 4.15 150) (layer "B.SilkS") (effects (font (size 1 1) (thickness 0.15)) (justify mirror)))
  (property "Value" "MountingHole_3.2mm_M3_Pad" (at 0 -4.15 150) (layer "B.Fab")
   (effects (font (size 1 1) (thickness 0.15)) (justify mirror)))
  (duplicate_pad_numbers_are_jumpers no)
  (pad "1" thru_hole circle (at 0 0 330) (size 6.4 6.4) (drill 3.2) (layers "*.Cu" "*.Mask") (remove_unused_layers no) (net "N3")
   (zone_connect 2)))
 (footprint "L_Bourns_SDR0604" (layer "B.Cu") (at 130.822114 66.022765 90)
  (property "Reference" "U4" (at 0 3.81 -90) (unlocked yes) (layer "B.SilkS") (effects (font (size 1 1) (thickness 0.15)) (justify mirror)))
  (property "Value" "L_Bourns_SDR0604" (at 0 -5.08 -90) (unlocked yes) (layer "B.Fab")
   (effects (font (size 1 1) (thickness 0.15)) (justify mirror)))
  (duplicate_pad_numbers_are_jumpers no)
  (pad "1" smd roundrect (at 0 1.95 90) (size 5.8 2.1) (layers "B.Cu" "B.Mask" "B.Paste") (roundrect_rratio 0) (chamfer_ratio 0.2)
   (chamfer bottom_left bottom_right) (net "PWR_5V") (die_length 2))
  (pad "2" smd roundrect (at 0 -1.95 270) (size 5.8 2.1) (layers "B.Cu" "B.Mask" "B.Paste") (roundrect_rratio 0) (chamfer_ratio 0.2)
   (chamfer bottom_left bottom_right) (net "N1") (die_length 2)))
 (gr_arc (start 100 54) (mid 101.171572 51.171572) (end 104 50) (stroke (width 0.05) (type default)) (layer "Edge.Cuts"))
 (gr_line (start 100 77.871446) (end 100 54) (stroke (width 0.05) (type default)) (layer "Edge.Cuts"))
 (gr_line (start 104 50) (end 148 50) (stroke (width 0.05) (type default)) (layer "Edge.Cuts"))
 (gr_arc (start 104 81.871446) (mid 101.171572 80.699873) (end 100 77.871446) (stroke (width 0.1) (type default)) (layer "Edge.Cuts"))
 (gr_circle (center 125.293536 56.65773) (end 127.293536 56.65773) (stroke (width 0.15) (type default)) (fill no) (layer "Edge.Cuts"))
 (gr_circle (center 138.215476 72.609354) (end 139.215476 72.609354) (stroke (width 0.15) (type default)) (fill no) (layer "Edge.Cuts"))
 (gr_arc (start 148 50) (mid 150.828427 51.171572) (end 152 54) (stroke (width 0.05) (type default)) (layer "Edge.Cuts"))
 (gr_line (start 148 81.871446) (end 104 81.871446) (stroke (width 0.15) (type default)) (layer "Edge.Cuts"))
 (gr_line (start 152 54) (end 152 77.871446) (stroke (width 0.15) (type default)) (layer "Edge.Cuts"))
 (gr_arc (start 152 77.871446) (mid 150.828427 80.699873) (end 148 81.871446) (stroke (width 0.15) (type default)) (layer "Edge.Cuts"))
 (via (at 140.495459 57.325445) (size 0.7) (drill 0.28) (layers "F.Cu" "B.Cu") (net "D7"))
 (segment (start 113.596447 65.696447) (end 108.596447 65.696447) (width 0.35) (layer "F.Cu") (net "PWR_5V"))
 (via (at 140.655417 61.055965) (size 0.8) (drill 0.4) (layers "F.Cu" "B.Cu") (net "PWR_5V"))
 (arc (start 113.95 65.55) (mid 113.787788 65.658386) (end 113.596447 65.696447) (width 0.35) (layer "F.Cu") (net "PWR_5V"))
 (segment (start 110.785668 72.262885) (end 115.785668 72.262885) (width 0.2) (layer "B.Cu") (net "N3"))
 (segment (start 109.515153 69.308399) (end 109.515153 70.308399) (width 0.35) (layer "B.Cu") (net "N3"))
 (segment (start 109.515153 70.308399) (end 109.515153 73.808399) (width 0.35) (layer "B.Cu") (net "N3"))
 (arc (start 108.929513 71.49404) (mid 109.781124 72.063068) (end 110.785668 72.262885) (width 0.2) (layer "B.Cu") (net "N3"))
 (segment (start 110.755391 69.150341) (end 110.755391 68.650341) (width 0.25) (layer "F.Cu") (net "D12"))
 (arc (start 109.380391 70.525341) (mid 110.352663 70.122613) (end 110.755391 69.150341) (width 0.25) (layer "F.Cu") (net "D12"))
 (arc (start 109.005391 70.150341) (mid 109.115226 70.415506) (end 109.380391 70.525341) (width 0.25) (layer "F.Cu") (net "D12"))
 (arc (start 108.822333 69.708399) (mid 108.957816 69.911164) (end 109.005391 70.150341) (width 0.25) (layer "F.Cu") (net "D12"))
 (segment (start 109.215813 65.65402) (end 109.215813 64.15402) (width 0.2) (layer "B.Cu") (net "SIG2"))
 (segment (start 112.286434 67.708399) (end 110.286434 67.708399) (width 0.2) (layer "B.Cu") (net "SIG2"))
 (arc (start 110.021269 67.598564) (mid 109.425144 66.7064) (end 109.215813 65.65402) (width 0.2) (layer "B.Cu") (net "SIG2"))
 (arc (start 110.286434 67.708399) (mid 110.142928 67.679854) (end 110.021269 67.598564) (width 0.2) (layer "B.Cu") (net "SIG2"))
 (via (at 136.054149 66.485149) (size 0.8) (drill 0.32) (layers "F.Cu" "B.Cu") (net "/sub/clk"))
 (segment (start 117.4 60.3) (end 119.4 58.3) (width 0.4) (layer "B.Cu") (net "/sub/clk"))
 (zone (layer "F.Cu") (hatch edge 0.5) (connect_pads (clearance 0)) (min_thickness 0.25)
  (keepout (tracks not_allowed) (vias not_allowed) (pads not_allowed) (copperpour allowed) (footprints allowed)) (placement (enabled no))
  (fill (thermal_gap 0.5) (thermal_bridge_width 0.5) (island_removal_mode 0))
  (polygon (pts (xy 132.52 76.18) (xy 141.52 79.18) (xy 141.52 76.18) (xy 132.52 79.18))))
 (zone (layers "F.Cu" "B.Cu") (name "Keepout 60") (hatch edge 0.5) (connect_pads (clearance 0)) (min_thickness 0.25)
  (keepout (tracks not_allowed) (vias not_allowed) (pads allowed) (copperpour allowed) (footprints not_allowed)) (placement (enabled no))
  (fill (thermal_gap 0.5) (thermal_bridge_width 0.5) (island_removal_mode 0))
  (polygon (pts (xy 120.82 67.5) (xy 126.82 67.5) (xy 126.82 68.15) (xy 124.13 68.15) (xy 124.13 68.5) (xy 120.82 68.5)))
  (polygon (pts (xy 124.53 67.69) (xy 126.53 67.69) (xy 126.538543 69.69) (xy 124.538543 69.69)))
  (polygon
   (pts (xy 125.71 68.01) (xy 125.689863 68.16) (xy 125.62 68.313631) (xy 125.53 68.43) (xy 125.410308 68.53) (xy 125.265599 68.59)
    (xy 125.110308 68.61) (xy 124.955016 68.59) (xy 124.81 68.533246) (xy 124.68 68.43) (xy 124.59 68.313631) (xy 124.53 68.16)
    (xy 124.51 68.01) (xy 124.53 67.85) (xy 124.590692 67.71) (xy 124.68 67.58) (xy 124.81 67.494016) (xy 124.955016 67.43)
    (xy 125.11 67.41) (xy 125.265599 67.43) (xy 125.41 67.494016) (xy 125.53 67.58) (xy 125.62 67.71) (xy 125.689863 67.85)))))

